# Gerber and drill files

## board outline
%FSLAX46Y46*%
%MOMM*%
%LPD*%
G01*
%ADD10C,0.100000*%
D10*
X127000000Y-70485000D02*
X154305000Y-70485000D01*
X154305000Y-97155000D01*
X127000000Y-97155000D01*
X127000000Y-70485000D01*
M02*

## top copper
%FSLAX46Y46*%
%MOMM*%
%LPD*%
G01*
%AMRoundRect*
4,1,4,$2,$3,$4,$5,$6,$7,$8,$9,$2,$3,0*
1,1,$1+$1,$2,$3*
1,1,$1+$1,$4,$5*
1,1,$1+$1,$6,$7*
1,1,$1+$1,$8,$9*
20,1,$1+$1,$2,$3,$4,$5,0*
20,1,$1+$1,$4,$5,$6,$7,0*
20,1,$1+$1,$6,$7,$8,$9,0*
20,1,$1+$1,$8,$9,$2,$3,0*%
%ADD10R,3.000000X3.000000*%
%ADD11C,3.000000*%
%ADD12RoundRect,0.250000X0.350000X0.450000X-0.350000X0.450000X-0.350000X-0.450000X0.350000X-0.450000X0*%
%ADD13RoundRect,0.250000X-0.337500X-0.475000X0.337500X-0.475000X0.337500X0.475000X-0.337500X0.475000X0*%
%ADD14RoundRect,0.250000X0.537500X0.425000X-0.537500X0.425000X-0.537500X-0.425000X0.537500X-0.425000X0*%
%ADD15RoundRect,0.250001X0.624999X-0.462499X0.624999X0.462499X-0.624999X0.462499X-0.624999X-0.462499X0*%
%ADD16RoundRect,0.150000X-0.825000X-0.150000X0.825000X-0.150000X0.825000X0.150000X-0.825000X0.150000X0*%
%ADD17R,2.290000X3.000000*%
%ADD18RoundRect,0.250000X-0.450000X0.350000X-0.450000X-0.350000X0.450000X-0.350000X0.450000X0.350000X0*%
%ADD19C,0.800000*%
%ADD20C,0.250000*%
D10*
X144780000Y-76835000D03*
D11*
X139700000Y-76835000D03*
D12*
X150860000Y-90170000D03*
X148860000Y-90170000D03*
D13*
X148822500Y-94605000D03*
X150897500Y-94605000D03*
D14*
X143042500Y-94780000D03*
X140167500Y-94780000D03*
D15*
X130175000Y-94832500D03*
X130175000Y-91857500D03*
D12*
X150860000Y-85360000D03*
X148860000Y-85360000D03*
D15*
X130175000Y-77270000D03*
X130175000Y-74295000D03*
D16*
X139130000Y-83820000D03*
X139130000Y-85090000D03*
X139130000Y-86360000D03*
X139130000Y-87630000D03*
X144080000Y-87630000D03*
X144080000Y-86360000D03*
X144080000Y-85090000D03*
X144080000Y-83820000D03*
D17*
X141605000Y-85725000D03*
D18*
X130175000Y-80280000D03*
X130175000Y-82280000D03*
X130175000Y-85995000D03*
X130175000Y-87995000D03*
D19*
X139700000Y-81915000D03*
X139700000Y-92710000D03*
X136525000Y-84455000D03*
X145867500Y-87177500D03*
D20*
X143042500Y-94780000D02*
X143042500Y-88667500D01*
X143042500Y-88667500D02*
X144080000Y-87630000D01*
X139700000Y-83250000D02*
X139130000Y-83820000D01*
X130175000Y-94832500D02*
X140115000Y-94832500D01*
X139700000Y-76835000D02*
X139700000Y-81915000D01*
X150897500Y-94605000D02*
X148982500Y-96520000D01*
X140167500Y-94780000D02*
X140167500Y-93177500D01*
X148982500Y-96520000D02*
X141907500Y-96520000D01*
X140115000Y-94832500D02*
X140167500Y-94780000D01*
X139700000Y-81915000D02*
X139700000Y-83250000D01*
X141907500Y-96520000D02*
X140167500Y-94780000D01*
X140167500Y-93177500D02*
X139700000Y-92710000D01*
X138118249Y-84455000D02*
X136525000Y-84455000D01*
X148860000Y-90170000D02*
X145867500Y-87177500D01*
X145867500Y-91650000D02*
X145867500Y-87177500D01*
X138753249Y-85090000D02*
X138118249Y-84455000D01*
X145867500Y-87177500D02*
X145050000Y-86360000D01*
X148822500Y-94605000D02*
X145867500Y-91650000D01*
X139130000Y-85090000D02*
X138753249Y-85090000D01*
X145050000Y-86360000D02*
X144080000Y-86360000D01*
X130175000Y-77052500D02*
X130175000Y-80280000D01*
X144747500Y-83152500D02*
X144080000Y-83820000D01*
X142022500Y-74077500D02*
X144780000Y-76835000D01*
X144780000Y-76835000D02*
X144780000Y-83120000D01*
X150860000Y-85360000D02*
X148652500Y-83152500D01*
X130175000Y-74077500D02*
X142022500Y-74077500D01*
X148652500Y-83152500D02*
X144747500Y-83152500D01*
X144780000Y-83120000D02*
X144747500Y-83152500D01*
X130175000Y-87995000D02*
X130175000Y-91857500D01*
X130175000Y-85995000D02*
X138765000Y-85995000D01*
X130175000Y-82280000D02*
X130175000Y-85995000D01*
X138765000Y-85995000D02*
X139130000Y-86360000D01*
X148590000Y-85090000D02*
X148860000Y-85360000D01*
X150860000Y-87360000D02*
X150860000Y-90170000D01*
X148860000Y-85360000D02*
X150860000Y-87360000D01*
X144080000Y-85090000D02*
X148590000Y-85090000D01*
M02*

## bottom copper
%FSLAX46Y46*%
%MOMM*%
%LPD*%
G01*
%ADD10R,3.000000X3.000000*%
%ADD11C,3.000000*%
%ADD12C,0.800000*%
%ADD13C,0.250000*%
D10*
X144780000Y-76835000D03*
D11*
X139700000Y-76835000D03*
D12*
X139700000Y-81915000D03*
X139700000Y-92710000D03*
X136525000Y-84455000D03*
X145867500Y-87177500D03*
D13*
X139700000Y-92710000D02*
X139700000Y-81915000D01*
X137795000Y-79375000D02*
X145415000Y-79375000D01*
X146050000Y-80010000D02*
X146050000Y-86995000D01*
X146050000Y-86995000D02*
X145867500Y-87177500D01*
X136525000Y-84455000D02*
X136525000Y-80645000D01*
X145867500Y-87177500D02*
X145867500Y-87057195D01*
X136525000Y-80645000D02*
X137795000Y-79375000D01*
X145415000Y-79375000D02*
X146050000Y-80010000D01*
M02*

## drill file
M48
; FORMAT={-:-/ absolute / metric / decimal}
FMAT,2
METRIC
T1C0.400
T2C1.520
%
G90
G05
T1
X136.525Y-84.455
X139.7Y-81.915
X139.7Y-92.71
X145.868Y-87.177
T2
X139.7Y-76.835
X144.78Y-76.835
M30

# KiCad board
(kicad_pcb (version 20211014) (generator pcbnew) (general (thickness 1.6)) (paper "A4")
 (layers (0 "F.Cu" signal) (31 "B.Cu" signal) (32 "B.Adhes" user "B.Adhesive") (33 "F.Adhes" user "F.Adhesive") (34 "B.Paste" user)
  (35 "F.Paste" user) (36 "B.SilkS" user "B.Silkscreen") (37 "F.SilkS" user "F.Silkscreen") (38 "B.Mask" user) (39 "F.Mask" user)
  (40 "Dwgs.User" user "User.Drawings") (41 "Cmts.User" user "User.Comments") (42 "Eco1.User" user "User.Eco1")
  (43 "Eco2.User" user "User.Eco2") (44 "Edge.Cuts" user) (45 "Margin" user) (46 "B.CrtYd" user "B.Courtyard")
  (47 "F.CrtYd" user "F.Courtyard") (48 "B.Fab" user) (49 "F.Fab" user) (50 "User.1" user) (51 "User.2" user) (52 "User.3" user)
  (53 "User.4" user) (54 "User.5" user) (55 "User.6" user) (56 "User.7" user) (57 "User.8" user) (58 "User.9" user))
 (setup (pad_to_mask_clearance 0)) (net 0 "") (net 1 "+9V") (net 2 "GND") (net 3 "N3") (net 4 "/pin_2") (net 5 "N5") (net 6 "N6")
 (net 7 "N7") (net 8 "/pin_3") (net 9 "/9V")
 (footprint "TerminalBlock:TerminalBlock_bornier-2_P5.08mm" (layer "F.Cu") (at 144.78 76.835 180)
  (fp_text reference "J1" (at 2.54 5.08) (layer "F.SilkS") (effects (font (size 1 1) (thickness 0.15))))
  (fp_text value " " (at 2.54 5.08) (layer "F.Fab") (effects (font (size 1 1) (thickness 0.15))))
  (pad "1" thru_hole rect (at 0 0 180) (size 3 3) (drill 1.52) (layers *.Cu *.Mask) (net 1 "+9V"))
  (pad "2" thru_hole circle (at 5.08 0 180) (size 3 3) (drill 1.52) (layers *.Cu *.Mask) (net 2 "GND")))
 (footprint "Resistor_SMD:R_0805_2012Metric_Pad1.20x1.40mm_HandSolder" (layer "F.Cu") (at 149.86 90.17 180)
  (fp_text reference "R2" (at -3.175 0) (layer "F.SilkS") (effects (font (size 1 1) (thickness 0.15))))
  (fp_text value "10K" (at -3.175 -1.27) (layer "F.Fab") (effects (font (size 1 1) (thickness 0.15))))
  (pad "1" smd roundrect (at -1 0 180) (size 1.2 1.4) (layers "F.Cu" "F.Paste" "F.Mask") (roundrect_rratio 0.2083333333) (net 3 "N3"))
  (pad "2" smd roundrect (at 1 0 180) (size 1.2 1.4) (layers "F.Cu" "F.Paste" "F.Mask") (roundrect_rratio 0.2083333333) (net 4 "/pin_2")))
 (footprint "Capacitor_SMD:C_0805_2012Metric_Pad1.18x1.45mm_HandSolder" (layer "F.Cu") (at 149.86 94.605)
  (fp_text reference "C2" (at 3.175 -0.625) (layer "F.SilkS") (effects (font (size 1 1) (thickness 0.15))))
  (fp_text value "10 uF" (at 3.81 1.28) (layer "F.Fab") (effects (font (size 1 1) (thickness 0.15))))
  (pad "2" smd roundrect (at -1.0375 0) (size 1.175 1.45) (layers "F.Cu" "F.Paste" "F.Mask") (roundrect_rratio 0.2127659574)
   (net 4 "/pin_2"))
  (pad "2" smd roundrect (at 1.0375 0) (size 1.175 1.45) (layers "F.Cu" "F.Paste" "F.Mask") (roundrect_rratio 0.2127659574) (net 2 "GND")))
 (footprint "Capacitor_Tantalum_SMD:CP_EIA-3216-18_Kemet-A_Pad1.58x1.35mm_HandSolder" (layer "F.Cu") (at 141.605 94.78 180)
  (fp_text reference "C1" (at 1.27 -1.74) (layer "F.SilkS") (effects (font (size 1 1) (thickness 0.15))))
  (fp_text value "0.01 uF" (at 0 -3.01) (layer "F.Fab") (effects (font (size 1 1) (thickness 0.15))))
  (pad "1" smd roundrect (at -1.4375 0 180) (size 1.575 1.35) (layers "F.Cu" "F.Paste" "F.Mask") (roundrect_rratio 0.1851851852)
   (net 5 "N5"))
  (pad "2" smd roundrect (at 1.4375 0 180) (size 1.575 1.35) (layers "F.Cu" "F.Paste" "F.Mask") (roundrect_rratio 0.1851851852)
   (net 2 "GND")))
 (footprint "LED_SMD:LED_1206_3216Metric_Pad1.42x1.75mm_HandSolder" (layer "F.Cu") (at 130.175 93.345 90)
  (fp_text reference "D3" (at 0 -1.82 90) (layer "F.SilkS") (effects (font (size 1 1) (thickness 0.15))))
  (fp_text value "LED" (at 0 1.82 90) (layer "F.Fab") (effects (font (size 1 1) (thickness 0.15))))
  (pad "1" smd roundrect (at -1.4875 0 90) (size 1.425 1.75) (layers "F.Cu" "F.Paste" "F.Mask") (roundrect_rratio 0.1754392982)
   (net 2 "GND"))
  (pad "2" smd roundrect (at 1.4875 0 90) (size 1.425 1.75) (layers "F.Cu" "F.Paste" "F.Mask") (roundrect_rratio 0.1754392982) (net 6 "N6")))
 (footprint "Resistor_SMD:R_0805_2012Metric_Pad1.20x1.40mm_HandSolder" (layer "F.Cu") (at 149.86 85.36 180)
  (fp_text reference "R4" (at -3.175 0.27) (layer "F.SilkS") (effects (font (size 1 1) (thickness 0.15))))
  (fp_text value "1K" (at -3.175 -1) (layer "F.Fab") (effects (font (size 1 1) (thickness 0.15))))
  (pad "1" smd roundrect (at -1 0 180) (size 1.2 1.4) (layers "F.Cu" "F.Paste" "F.Mask") (roundrect_rratio 0.2083333333) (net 1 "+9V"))
  (pad "2" smd roundrect (at 1 0 180) (size 1.2 1.4) (layers "F.Cu" "F.Paste" "F.Mask") (roundrect_rratio 0.2083333333) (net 3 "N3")))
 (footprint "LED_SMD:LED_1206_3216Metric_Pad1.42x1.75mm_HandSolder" (layer "F.Cu") (at 130.175 75.7825 90)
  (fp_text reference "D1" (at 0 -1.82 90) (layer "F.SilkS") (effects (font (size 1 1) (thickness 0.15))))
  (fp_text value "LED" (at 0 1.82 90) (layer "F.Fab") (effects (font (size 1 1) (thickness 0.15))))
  (pad "1" smd roundrect (at -1.4875 0 90) (size 1.425 1.75) (layers "F.Cu" "F.Paste" "F.Mask") (roundrect_rratio 0.1754392982) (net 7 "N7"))
  (pad "2" smd roundrect (at 1.4875 0 90) (size 1.425 1.75) (layers "F.Cu" "F.Paste" "F.Mask") (roundrect_rratio 0.1754392982) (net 1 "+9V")))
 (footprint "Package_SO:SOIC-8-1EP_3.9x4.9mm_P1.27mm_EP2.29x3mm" (layer "F.Cu") (at 141.605 85.725)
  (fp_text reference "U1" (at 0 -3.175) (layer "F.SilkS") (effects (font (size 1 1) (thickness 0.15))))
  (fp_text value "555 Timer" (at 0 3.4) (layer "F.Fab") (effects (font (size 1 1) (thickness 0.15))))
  (pad "" smd roundrect (at 0.57 -0.75) (size 0.92 1.21) (layers "F.Paste") (roundrect_rratio 0.25))
  (pad "" smd roundrect (at 0.57 0.75) (size 0.92 1.21) (layers "F.Paste") (roundrect_rratio 0.25))
  (pad "" smd roundrect (at -0.57 0.75) (size 0.92 1.21) (layers "F.Paste") (roundrect_rratio 0.25))
  (pad "" smd roundrect (at -0.57 -0.75) (size 0.92 1.21) (layers "F.Paste") (roundrect_rratio 0.25))
  (pad "1" smd roundrect (at -2.475 -1.905) (size 1.95 0.6) (layers "F.Cu" "F.Paste" "F.Mask") (roundrect_rratio 0.25) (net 2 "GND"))
  (pad "2" smd roundrect (at -2.475 -0.635) (size 1.95 0.6) (layers "F.Cu" "F.Paste" "F.Mask") (roundrect_rratio 0.25) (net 4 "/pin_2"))
  (pad "3" smd roundrect (at -2.475 0.635) (size 1.95 0.6) (layers "F.Cu" "F.Paste" "F.Mask") (roundrect_rratio 0.25) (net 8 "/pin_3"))
  (pad "4" smd roundrect (at -2.475 1.905) (size 1.95 0.6) (layers "F.Cu" "F.Paste" "F.Mask") (roundrect_rratio 0.25) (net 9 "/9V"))
  (pad "5" smd roundrect (at 2.475 1.905) (size 1.95 0.6) (layers "F.Cu" "F.Paste" "F.Mask") (roundrect_rratio 0.25) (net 5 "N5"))
  (pad "6" smd roundrect (at 2.475 0.635) (size 1.95 0.6) (layers "F.Cu" "F.Paste" "F.Mask") (roundrect_rratio 0.25) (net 4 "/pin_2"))
  (pad "7" smd roundrect (at 2.475 -0.635) (size 1.95 0.6) (layers "F.Cu" "F.Paste" "F.Mask") (roundrect_rratio 0.25) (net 3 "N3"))
  (pad "8" smd roundrect (at 2.475 -1.905) (size 1.95 0.6) (layers "F.Cu" "F.Paste" "F.Mask") (roundrect_rratio 0.25) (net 1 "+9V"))
  (pad "9" smd rect (at 0 0) (size 2.29 3) (layers "F.Cu" "F.Mask")))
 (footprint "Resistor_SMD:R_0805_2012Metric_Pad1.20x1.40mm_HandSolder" (layer "F.Cu") (at 130.175 81.28 -90)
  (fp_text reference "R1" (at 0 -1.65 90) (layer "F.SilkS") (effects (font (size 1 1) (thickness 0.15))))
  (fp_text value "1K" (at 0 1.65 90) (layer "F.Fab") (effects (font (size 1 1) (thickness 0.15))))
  (pad "1" smd roundrect (at -1 0 270) (size 1.2 1.4) (layers "F.Cu" "F.Paste" "F.Mask") (roundrect_rratio 0.2083333333) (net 7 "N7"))
  (pad "2" smd roundrect (at 1 0 270) (size 1.2 1.4) (layers "F.Cu" "F.Paste" "F.Mask") (roundrect_rratio 0.2083333333) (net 8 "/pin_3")))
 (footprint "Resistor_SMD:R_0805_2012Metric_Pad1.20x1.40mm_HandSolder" (layer "F.Cu") (at 130.175 86.995 -90)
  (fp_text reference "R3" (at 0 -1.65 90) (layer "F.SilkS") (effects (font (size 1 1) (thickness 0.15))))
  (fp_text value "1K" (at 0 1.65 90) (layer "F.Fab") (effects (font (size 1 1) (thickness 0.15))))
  (pad "1" smd roundrect (at -1 0 270) (size 1.2 1.4) (layers "F.Cu" "F.Paste" "F.Mask") (roundrect_rratio 0.2083333333) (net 8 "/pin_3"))
  (pad "2" smd roundrect (at 1 0 270) (size 1.2 1.4) (layers "F.Cu" "F.Paste" "F.Mask") (roundrect_rratio 0.2083333333) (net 6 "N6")))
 (gr_rect (start 127 70.485) (end 154.305 97.155) (layer "Edge.Cuts") (width 0.1) (fill none))
 (segment (start 143.0425 94.78) (end 143.0425 88.6675) (width 0.25) (layer "F.Cu") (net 5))
 (segment (start 143.0425 88.6675) (end 144.08 87.63) (width 0.25) (layer "F.Cu") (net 5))
 (segment (start 139.7 83.25) (end 139.13 83.82) (width 0.25) (layer "F.Cu") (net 2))
 (segment (start 130.175 94.8325) (end 140.115 94.8325) (width 0.25) (layer "F.Cu") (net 2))
 (segment (start 139.7 76.835) (end 139.7 81.915) (width 0.25) (layer "F.Cu") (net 2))
 (segment (start 150.8975 94.605) (end 148.9825 96.52) (width 0.25) (layer "F.Cu") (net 2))
 (segment (start 140.1675 94.78) (end 140.1675 93.1775) (width 0.25) (layer "F.Cu") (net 2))
 (segment (start 148.9825 96.52) (end 141.9075 96.52) (width 0.25) (layer "F.Cu") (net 2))
 (segment (start 140.115 94.8325) (end 140.1675 94.78) (width 0.25) (layer "F.Cu") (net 2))
 (segment (start 139.7 81.915) (end 139.7 83.25) (width 0.25) (layer "F.Cu") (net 2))
 (segment (start 141.9075 96.52) (end 140.1675 94.78) (width 0.25) (layer "F.Cu") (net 2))
 (segment (start 140.1675 93.1775) (end 139.7 92.71) (width 0.25) (layer "F.Cu") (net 2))
 (via (at 139.7 81.915) (size 0.8) (drill 0.4) (layers "F.Cu" "B.Cu") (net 2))
 (via (at 139.7 92.71) (size 0.8) (drill 0.4) (layers "F.Cu" "B.Cu") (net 2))
 (segment (start 139.7 92.71) (end 139.7 81.915) (width 0.25) (layer "B.Cu") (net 2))
 (segment (start 138.118249 84.455) (end 136.525 84.455) (width 0.25) (layer "F.Cu") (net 4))
 (segment (start 148.86 90.17) (end 145.8675 87.1775) (width 0.25) (layer "F.Cu") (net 4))
 (segment (start 145.8675 91.65) (end 145.8675 87.1775) (width 0.25) (layer "F.Cu") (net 4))
 (segment (start 138.753249 85.09) (end 138.118249 84.455) (width 0.25) (layer "F.Cu") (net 4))
 (segment (start 145.8675 87.1775) (end 145.05 86.36) (width 0.25) (layer "F.Cu") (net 4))
 (segment (start 148.8225 94.605) (end 145.8675 91.65) (width 0.25) (layer "F.Cu") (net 4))
 (segment (start 139.13 85.09) (end 138.753249 85.09) (width 0.25) (layer "F.Cu") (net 4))
 (segment (start 145.05 86.36) (end 144.08 86.36) (width 0.25) (layer "F.Cu") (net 4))
 (via (at 136.525 84.455) (size 0.8) (drill 0.4) (layers "F.Cu" "B.Cu") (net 4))
 (via (at 145.8675 87.1775) (size 0.8) (drill 0.4) (layers "F.Cu" "B.Cu") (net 4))
 (segment (start 137.795 79.375) (end 145.415 79.375) (width 0.25) (layer "B.Cu") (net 4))
 (segment (start 146.05 80.01) (end 146.05 86.995) (width 0.25) (layer "B.Cu") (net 4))
 (segment (start 146.05 86.995) (end 145.8675 87.1775) (width 0.25) (layer "B.Cu") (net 4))
 (segment (start 136.525 84.455) (end 136.525 80.645) (width 0.25) (layer "B.Cu") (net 4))
 (segment (start 145.8675 87.1775) (end 145.8675 87.057195) (width 0.25) (layer "B.Cu") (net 4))
 (segment (start 136.525 80.645) (end 137.795 79.375) (width 0.25) (layer "B.Cu") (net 4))
 (segment (start 145.415 79.375) (end 146.05 80.01) (width 0.25) (layer "B.Cu") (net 4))
 (segment (start 130.175 77.0525) (end 130.175 80.28) (width 0.25) (layer "F.Cu") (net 7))
 (segment (start 144.7475 83.1525) (end 144.08 83.82) (width 0.25) (layer "F.Cu") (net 1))
 (segment (start 142.0225 74.0775) (end 144.78 76.835) (width 0.25) (layer "F.Cu") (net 1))
 (segment (start 144.78 76.835) (end 144.78 83.12) (width 0.25) (layer "F.Cu") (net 1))
 (segment (start 150.86 85.36) (end 148.6525 83.1525) (width 0.25) (layer "F.Cu") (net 1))
 (segment (start 130.175 74.0775) (end 142.0225 74.0775) (width 0.25) (layer "F.Cu") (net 1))
 (segment (start 148.6525 83.1525) (end 144.7475 83.1525) (width 0.25) (layer "F.Cu") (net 1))
 (segment (start 144.78 83.12) (end 144.7475 83.1525) (width 0.25) (layer "F.Cu") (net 1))
 (segment (start 130.175 87.995) (end 130.175 91.8575) (width 0.25) (layer "F.Cu") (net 6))
 (segment (start 130.175 85.995) (end 138.765 85.995) (width 0.25) (layer "F.Cu") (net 8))
 (segment (start 130.175 82.28) (end 130.175 85.995) (width 0.25) (layer "F.Cu") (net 8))
 (segment (start 138.765 85.995) (end 139.13 86.36) (width 0.25) (layer "F.Cu") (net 8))
 (segment (start 148.59 85.09) (end 148.86 85.36) (width 0.25) (layer "F.Cu") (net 3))
 (segment (start 150.86 87.36) (end 150.86 90.17) (width 0.25) (layer "F.Cu") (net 3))
 (segment (start 148.86 85.36) (end 150.86 87.36) (width 0.25) (layer "F.Cu") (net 3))
 (segment (start 144.08 85.09) (end 148.59 85.09) (width 0.25) (layer "F.Cu") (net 3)))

